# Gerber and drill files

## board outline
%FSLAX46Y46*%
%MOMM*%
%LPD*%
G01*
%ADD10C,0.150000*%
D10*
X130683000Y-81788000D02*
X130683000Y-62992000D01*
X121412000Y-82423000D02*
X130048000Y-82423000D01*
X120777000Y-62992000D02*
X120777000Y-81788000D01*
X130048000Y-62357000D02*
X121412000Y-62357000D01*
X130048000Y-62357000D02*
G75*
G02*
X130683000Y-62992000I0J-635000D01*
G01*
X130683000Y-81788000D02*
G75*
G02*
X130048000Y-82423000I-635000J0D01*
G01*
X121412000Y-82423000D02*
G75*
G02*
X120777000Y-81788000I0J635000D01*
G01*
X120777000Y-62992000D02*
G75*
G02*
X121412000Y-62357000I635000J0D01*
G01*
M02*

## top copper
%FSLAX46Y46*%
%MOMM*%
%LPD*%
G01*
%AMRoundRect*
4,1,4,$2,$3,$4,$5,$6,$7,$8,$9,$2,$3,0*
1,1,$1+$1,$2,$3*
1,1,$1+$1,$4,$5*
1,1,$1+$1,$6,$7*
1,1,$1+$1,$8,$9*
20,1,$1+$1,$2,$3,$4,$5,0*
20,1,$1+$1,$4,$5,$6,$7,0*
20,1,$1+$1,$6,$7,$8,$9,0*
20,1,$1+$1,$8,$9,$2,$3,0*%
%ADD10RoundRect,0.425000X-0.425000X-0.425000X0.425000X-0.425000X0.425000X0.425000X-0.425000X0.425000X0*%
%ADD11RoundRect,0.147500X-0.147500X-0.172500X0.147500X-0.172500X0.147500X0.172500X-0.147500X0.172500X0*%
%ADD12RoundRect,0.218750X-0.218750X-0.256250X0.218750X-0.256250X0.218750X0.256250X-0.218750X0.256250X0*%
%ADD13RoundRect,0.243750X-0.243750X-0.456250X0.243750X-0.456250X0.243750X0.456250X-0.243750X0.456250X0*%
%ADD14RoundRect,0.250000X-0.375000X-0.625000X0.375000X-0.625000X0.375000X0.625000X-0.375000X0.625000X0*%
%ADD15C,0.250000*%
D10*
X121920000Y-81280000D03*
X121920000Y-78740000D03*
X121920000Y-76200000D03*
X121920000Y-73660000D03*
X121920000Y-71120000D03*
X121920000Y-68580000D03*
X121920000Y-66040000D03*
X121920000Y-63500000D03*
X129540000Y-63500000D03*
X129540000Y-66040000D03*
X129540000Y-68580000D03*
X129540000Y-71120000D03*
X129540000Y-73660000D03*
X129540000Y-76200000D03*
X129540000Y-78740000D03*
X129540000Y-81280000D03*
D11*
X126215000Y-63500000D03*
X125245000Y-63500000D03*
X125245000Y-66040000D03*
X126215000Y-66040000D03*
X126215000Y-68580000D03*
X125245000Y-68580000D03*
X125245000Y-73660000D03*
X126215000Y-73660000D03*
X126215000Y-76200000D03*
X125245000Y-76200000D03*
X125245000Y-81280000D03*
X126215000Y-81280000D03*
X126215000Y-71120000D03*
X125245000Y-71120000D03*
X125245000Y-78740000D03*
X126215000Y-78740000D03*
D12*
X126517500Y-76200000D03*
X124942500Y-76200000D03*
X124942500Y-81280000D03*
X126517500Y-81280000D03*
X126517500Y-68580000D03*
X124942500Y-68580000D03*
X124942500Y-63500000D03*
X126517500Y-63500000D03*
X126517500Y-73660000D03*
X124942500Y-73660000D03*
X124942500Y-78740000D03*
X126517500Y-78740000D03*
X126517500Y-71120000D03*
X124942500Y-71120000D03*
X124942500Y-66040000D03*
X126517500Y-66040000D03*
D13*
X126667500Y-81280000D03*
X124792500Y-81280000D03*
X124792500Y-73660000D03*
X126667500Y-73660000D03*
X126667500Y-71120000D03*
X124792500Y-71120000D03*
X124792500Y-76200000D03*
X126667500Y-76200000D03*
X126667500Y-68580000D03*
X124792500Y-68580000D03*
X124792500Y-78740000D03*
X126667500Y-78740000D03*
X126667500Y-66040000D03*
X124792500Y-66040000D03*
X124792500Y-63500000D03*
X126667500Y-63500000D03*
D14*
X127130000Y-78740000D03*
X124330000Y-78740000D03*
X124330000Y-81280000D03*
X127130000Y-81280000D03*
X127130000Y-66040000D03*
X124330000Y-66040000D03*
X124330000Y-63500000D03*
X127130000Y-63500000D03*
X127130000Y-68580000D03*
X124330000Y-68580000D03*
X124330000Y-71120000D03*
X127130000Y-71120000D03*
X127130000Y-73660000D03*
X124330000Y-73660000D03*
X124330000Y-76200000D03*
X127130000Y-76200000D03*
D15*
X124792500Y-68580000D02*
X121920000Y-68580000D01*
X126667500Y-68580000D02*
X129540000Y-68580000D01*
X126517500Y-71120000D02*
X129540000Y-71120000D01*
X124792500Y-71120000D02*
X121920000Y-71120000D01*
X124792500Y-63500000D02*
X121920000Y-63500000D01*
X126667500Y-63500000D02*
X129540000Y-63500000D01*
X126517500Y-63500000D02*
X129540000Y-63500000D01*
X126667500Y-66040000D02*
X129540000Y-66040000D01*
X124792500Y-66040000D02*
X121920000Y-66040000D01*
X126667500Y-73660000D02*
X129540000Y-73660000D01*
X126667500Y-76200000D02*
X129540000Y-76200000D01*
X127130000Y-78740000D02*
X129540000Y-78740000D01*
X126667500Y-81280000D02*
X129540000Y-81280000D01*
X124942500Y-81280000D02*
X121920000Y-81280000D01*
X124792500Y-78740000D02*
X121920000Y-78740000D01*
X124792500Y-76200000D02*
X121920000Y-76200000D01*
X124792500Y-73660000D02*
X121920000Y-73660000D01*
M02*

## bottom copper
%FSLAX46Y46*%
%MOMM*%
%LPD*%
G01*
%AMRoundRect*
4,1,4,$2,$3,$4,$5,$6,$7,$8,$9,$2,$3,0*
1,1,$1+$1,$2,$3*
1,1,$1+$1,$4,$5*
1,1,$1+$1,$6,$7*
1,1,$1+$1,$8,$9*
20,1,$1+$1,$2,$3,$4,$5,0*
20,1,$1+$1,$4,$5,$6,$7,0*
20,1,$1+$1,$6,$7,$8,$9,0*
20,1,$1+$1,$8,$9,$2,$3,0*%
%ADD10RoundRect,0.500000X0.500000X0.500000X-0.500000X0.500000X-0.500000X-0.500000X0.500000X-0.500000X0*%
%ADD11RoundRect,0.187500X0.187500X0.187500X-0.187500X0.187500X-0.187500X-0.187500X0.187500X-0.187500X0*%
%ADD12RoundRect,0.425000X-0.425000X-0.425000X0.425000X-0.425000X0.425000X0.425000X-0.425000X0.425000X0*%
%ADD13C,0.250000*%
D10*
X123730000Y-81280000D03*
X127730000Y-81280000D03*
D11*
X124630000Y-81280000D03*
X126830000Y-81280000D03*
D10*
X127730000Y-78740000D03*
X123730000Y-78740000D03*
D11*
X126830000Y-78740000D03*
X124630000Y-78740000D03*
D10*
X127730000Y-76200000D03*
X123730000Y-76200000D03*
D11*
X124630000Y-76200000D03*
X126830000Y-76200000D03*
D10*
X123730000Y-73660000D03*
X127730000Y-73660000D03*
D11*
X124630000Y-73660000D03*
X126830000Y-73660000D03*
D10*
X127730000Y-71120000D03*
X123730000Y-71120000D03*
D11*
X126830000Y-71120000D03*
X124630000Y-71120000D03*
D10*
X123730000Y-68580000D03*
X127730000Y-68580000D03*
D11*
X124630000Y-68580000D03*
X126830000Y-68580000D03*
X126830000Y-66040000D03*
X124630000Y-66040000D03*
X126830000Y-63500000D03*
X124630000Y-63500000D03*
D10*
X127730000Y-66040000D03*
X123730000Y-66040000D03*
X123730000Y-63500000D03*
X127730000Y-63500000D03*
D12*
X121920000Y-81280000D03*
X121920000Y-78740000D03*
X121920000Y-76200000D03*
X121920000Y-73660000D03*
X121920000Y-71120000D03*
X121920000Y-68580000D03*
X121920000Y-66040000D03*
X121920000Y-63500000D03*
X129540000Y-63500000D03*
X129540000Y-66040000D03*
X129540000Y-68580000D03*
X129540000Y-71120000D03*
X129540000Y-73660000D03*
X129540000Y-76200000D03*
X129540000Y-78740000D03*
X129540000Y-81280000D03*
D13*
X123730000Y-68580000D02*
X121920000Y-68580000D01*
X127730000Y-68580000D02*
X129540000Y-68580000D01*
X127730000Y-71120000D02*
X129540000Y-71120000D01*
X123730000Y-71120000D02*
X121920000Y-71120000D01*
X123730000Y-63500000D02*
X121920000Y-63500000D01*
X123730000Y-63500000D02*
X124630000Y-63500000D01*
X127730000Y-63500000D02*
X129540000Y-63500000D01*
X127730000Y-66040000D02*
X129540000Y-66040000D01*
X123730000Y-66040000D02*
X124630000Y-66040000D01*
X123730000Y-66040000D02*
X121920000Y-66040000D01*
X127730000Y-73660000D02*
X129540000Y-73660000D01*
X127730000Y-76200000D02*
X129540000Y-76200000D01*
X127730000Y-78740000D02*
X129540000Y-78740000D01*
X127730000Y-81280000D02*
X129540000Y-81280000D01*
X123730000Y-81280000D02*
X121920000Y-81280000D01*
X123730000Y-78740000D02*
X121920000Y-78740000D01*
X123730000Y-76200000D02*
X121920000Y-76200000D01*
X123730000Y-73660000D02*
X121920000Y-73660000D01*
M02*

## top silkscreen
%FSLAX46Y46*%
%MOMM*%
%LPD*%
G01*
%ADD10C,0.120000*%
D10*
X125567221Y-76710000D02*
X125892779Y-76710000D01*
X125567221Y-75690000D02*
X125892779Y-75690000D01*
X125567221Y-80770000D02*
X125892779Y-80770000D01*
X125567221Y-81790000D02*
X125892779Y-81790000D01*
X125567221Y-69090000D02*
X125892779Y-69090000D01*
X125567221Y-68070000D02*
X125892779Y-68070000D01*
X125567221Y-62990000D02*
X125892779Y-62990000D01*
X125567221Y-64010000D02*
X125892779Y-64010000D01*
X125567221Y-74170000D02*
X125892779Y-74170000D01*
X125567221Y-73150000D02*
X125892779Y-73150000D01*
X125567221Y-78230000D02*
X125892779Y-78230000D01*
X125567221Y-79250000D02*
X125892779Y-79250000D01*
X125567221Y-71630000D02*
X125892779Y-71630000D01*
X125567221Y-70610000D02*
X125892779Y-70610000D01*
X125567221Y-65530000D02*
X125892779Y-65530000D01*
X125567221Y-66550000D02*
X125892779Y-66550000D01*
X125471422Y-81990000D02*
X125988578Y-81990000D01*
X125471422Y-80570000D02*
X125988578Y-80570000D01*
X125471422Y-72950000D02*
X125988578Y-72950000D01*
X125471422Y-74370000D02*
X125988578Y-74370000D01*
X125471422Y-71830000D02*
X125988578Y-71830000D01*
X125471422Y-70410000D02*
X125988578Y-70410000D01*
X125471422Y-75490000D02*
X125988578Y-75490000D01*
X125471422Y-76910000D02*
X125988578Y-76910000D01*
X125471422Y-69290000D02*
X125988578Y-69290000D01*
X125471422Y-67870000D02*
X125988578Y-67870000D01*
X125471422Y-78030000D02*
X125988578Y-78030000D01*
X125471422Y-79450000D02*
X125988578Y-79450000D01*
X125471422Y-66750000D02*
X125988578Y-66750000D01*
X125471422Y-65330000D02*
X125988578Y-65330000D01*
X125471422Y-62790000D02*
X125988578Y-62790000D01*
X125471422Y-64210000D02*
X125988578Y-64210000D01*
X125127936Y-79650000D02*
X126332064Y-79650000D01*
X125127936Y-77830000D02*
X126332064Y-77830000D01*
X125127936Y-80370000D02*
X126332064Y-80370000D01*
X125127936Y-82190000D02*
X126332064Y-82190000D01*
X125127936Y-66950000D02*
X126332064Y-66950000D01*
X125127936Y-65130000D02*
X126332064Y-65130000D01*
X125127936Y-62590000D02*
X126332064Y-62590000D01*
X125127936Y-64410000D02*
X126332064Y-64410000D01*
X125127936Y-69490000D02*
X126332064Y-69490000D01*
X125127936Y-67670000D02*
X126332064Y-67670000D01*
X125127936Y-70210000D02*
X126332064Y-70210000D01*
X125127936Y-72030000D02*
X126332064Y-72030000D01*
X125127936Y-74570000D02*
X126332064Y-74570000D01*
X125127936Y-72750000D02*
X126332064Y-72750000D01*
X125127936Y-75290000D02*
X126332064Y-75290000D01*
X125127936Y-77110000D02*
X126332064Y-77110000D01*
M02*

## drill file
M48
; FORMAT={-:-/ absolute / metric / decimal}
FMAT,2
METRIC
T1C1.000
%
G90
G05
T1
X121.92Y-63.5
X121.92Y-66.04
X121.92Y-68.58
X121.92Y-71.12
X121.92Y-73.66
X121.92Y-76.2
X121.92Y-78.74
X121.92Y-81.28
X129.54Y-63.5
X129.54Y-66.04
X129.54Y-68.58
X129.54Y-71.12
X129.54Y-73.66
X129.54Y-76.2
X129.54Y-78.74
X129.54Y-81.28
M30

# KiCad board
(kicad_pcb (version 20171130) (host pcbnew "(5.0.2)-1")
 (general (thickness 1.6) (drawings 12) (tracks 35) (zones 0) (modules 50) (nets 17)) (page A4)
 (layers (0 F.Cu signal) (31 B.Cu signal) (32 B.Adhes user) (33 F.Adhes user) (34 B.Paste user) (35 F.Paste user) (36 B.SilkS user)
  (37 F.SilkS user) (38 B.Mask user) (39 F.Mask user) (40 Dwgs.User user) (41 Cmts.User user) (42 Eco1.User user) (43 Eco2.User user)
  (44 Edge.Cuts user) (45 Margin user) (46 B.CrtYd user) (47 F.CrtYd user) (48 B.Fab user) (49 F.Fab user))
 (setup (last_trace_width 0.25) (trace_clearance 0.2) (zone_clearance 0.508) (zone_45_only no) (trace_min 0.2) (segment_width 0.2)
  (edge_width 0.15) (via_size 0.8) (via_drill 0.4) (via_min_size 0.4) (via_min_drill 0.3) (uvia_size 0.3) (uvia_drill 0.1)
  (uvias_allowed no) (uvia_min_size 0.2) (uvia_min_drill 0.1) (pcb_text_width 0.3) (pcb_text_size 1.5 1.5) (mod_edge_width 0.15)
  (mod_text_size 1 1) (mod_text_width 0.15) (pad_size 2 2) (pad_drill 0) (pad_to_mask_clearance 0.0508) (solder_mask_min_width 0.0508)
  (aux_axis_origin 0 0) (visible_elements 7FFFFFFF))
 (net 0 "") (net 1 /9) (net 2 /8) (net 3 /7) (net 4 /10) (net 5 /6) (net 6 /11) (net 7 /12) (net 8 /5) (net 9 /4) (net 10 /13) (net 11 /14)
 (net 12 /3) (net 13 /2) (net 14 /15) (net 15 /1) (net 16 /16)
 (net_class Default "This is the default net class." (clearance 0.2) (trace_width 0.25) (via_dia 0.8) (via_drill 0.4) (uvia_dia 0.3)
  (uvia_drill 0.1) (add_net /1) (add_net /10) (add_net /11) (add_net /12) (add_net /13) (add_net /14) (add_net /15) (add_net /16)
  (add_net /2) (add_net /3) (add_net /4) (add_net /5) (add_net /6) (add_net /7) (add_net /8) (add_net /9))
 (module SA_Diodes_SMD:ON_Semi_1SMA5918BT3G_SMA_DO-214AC (layer B.Cu) (at 125.73 81.28 180)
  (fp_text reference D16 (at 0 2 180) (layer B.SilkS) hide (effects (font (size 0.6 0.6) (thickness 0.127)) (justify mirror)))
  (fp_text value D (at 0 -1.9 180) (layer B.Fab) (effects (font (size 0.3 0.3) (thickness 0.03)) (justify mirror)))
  (pad 2 smd roundrect (at 2 0 180) (size 2 2) (layers B.Cu B.Paste B.Mask) (roundrect_rratio 0.25) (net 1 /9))
  (pad 1 smd roundrect (at -2 0 180) (size 2 2) (layers B.Cu B.Paste B.Mask) (roundrect_rratio 0.25) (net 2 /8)))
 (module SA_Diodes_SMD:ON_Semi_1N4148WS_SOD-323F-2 (layer B.Cu) (at 125.73 81.28 180)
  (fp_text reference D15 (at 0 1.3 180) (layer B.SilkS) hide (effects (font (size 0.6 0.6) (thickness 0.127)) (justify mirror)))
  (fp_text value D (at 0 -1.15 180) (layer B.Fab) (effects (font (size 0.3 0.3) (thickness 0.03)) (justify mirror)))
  (pad 2 smd roundrect (at 1.1 0 180) (size 0.75 0.75) (layers B.Cu B.Paste B.Mask) (roundrect_rratio 0.25) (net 1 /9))
  (pad 1 smd roundrect (at -1.1 0 180) (size 0.75 0.75) (layers B.Cu B.Paste B.Mask) (roundrect_rratio 0.25) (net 2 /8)))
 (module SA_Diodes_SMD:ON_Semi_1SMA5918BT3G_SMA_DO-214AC (layer B.Cu) (at 125.73 78.74 180)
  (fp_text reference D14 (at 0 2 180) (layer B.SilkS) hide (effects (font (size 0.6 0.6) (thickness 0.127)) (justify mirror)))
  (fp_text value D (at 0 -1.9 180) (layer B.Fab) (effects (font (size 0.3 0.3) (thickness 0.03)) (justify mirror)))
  (pad 1 smd roundrect (at -2 0 180) (size 2 2) (layers B.Cu B.Paste B.Mask) (roundrect_rratio 0.25) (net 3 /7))
  (pad 2 smd roundrect (at 2 0 180) (size 2 2) (layers B.Cu B.Paste B.Mask) (roundrect_rratio 0.25) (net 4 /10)))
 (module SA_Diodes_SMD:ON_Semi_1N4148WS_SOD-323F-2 (layer B.Cu) (at 125.73 78.74 180)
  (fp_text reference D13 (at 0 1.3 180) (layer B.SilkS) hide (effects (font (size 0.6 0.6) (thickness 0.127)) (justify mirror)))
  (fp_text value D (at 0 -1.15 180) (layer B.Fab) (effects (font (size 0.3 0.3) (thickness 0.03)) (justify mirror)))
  (pad 1 smd roundrect (at -1.1 0 180) (size 0.75 0.75) (layers B.Cu B.Paste B.Mask) (roundrect_rratio 0.25) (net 3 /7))
  (pad 2 smd roundrect (at 1.1 0 180) (size 0.75 0.75) (layers B.Cu B.Paste B.Mask) (roundrect_rratio 0.25) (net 4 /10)))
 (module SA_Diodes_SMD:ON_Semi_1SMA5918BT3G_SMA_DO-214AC (layer B.Cu) (at 125.73 76.2 180)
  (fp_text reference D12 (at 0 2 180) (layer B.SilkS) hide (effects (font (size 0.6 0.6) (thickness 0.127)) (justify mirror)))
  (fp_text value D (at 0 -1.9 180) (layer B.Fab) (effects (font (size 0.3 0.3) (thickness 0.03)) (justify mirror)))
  (pad 1 smd roundrect (at -2 0 180) (size 2 2) (layers B.Cu B.Paste B.Mask) (roundrect_rratio 0.25) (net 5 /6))
  (pad 2 smd roundrect (at 2 0 180) (size 2 2) (layers B.Cu B.Paste B.Mask) (roundrect_rratio 0.25) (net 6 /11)))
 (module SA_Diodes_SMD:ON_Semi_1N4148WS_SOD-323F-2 (layer B.Cu) (at 125.73 76.2 180)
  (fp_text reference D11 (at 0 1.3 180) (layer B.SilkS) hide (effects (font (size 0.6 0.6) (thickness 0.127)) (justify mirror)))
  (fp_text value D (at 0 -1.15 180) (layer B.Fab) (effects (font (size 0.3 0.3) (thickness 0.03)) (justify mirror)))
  (pad 2 smd roundrect (at 1.1 0 180) (size 0.75 0.75) (layers B.Cu B.Paste B.Mask) (roundrect_rratio 0.25) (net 6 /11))
  (pad 1 smd roundrect (at -1.1 0 180) (size 0.75 0.75) (layers B.Cu B.Paste B.Mask) (roundrect_rratio 0.25) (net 5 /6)))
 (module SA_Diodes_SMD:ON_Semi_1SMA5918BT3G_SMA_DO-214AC (layer B.Cu) (at 125.73 73.66 180)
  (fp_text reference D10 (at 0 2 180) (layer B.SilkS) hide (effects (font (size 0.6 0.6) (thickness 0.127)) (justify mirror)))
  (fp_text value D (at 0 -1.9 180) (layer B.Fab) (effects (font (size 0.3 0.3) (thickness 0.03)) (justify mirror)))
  (pad 2 smd roundrect (at 2 0 180) (size 2 2) (layers B.Cu B.Paste B.Mask) (roundrect_rratio 0.25) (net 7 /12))
  (pad 1 smd roundrect (at -2 0 180) (size 2 2) (layers B.Cu B.Paste B.Mask) (roundrect_rratio 0.25) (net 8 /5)))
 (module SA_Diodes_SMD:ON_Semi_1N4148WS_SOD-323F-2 (layer B.Cu) (at 125.73 73.66 180)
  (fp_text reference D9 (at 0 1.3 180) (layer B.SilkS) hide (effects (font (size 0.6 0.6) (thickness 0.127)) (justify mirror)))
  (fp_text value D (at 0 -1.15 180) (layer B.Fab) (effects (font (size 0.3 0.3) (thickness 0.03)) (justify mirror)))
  (pad 2 smd roundrect (at 1.1 0 180) (size 0.75 0.75) (layers B.Cu B.Paste B.Mask) (roundrect_rratio 0.25) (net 7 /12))
  (pad 1 smd roundrect (at -1.1 0 180) (size 0.75 0.75) (layers B.Cu B.Paste B.Mask) (roundrect_rratio 0.25) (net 8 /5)))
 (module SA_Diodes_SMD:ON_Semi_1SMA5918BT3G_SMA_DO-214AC (layer B.Cu) (at 125.73 71.12 180)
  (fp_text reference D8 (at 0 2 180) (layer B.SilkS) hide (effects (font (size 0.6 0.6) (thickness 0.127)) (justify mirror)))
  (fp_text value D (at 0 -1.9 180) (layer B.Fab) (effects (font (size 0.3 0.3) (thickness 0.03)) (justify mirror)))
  (pad 1 smd roundrect (at -2 0 180) (size 2 2) (layers B.Cu B.Paste B.Mask) (roundrect_rratio 0.25) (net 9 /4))
  (pad 2 smd roundrect (at 2 0 180) (size 2 2) (layers B.Cu B.Paste B.Mask) (roundrect_rratio 0.25) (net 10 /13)))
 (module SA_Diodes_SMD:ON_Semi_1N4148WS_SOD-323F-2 (layer B.Cu) (at 125.73 71.12 180)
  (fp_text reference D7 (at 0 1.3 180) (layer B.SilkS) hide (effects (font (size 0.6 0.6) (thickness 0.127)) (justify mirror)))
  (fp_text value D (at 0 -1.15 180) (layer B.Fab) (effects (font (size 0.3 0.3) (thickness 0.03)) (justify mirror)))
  (pad 1 smd roundrect (at -1.1 0 180) (size 0.75 0.75) (layers B.Cu B.Paste B.Mask) (roundrect_rratio 0.25) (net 9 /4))
  (pad 2 smd roundrect (at 1.1 0 180) (size 0.75 0.75) (layers B.Cu B.Paste B.Mask) (roundrect_rratio 0.25) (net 10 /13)))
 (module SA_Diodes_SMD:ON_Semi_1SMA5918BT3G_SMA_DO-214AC (layer B.Cu) (at 125.73 68.58 180)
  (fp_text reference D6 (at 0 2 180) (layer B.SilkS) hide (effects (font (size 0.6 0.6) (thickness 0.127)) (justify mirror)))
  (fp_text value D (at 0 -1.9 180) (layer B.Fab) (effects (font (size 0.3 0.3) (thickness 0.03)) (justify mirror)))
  (pad 2 smd roundrect (at 2 0 180) (size 2 2) (layers B.Cu B.Paste B.Mask) (roundrect_rratio 0.25) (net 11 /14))
  (pad 1 smd roundrect (at -2 0 180) (size 2 2) (layers B.Cu B.Paste B.Mask) (roundrect_rratio 0.25) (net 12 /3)))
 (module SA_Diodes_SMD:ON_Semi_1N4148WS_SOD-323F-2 (layer B.Cu) (at 125.73 68.58 180)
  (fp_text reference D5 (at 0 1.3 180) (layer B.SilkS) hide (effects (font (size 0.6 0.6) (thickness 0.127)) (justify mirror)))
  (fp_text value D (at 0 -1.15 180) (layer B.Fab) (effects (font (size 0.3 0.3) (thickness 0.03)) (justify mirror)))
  (pad 2 smd roundrect (at 1.1 0 180) (size 0.75 0.75) (layers B.Cu B.Paste B.Mask) (roundrect_rratio 0.25) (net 11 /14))
  (pad 1 smd roundrect (at -1.1 0 180) (size 0.75 0.75) (layers B.Cu B.Paste B.Mask) (roundrect_rratio 0.25) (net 12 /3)))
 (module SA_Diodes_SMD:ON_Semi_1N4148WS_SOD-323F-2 (layer B.Cu) (at 125.73 66.04 180)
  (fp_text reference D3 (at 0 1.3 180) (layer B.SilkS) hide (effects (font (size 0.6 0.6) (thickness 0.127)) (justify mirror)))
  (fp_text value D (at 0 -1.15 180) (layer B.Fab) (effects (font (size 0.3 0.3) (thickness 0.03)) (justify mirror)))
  (pad 1 smd roundrect (at -1.1 0 180) (size 0.75 0.75) (layers B.Cu B.Paste B.Mask) (roundrect_rratio 0.25) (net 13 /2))
  (pad 2 smd roundrect (at 1.1 0 180) (size 0.75 0.75) (layers B.Cu B.Paste B.Mask) (roundrect_rratio 0.25) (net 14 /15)))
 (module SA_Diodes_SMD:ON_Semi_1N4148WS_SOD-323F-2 (layer B.Cu) (at 125.73 63.5 180)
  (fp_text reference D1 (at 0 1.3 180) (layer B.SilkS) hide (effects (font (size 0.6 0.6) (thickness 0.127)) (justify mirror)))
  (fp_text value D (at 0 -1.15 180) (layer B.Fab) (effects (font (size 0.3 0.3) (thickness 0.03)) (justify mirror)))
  (pad 1 smd roundrect (at -1.1 0 180) (size 0.75 0.75) (layers B.Cu B.Paste B.Mask) (roundrect_rratio 0.25) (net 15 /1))
  (pad 2 smd roundrect (at 1.1 0 180) (size 0.75 0.75) (layers B.Cu B.Paste B.Mask) (roundrect_rratio 0.25) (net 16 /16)))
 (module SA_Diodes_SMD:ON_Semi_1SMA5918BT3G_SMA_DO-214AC (layer B.Cu) (at 125.73 66.04 180)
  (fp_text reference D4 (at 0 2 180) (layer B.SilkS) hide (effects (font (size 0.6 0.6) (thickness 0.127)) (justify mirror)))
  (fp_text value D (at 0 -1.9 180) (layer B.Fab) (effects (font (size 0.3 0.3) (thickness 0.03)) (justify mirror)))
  (pad 1 smd roundrect (at -2 0 180) (size 2 2) (layers B.Cu B.Paste B.Mask) (roundrect_rratio 0.25) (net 13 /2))
  (pad 2 smd roundrect (at 2 0 180) (size 2 2) (layers B.Cu B.Paste B.Mask) (roundrect_rratio 0.25) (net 14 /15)))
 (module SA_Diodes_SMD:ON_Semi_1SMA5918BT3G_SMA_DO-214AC (layer B.Cu) (at 125.73 63.5 180)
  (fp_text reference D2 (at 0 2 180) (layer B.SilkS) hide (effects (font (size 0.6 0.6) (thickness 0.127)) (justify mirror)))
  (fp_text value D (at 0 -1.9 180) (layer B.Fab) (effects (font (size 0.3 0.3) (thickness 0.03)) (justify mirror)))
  (pad 2 smd roundrect (at 2 0 180) (size 2 2) (layers B.Cu B.Paste B.Mask) (roundrect_rratio 0.25) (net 16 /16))
  (pad 1 smd roundrect (at -2 0 180) (size 2 2) (layers B.Cu B.Paste B.Mask) (roundrect_rratio 0.25) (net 15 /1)))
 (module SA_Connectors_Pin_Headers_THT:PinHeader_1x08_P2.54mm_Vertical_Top (layer F.Cu) (at 121.92 63.5)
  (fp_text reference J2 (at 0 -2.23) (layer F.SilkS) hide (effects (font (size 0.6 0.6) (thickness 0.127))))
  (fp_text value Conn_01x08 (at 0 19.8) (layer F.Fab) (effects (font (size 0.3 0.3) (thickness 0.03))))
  (pad 8 thru_hole roundrect (at 0 17.78) (size 1.7 1.7) (drill 1) (layers *.Cu *.Mask) (roundrect_rratio 0.25) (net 1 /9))
  (pad 7 thru_hole roundrect (at 0 15.24) (size 1.7 1.7) (drill 1) (layers *.Cu *.Mask) (roundrect_rratio 0.25) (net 4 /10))
  (pad 6 thru_hole roundrect (at 0 12.7) (size 1.7 1.7) (drill 1) (layers *.Cu *.Mask) (roundrect_rratio 0.25) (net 6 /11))
  (pad 5 thru_hole roundrect (at 0 10.16) (size 1.7 1.7) (drill 1) (layers *.Cu *.Mask) (roundrect_rratio 0.25) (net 7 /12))
  (pad 4 thru_hole roundrect (at 0 7.62) (size 1.7 1.7) (drill 1) (layers *.Cu *.Mask) (roundrect_rratio 0.25) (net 10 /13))
  (pad 3 thru_hole roundrect (at 0 5.08) (size 1.7 1.7) (drill 1) (layers *.Cu *.Mask) (roundrect_rratio 0.25) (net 11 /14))
  (pad 2 thru_hole roundrect (at 0 2.54) (size 1.7 1.7) (drill 1) (layers *.Cu *.Mask) (roundrect_rratio 0.25) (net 14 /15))
  (pad 1 thru_hole roundrect (at 0 0) (size 1.7 1.7) (drill 1) (layers *.Cu *.Mask) (roundrect_rratio 0.25) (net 16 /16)))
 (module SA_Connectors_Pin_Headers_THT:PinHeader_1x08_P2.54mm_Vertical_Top (layer F.Cu) (at 129.54 63.5)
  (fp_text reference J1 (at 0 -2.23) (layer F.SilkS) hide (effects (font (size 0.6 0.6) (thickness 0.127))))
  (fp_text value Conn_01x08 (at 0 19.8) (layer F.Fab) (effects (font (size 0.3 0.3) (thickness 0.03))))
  (pad 1 thru_hole roundrect (at 0 0) (size 1.7 1.7) (drill 1) (layers *.Cu *.Mask) (roundrect_rratio 0.25) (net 15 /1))
  (pad 2 thru_hole roundrect (at 0 2.54) (size 1.7 1.7) (drill 1) (layers *.Cu *.Mask) (roundrect_rratio 0.25) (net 13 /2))
  (pad 3 thru_hole roundrect (at 0 5.08) (size 1.7 1.7) (drill 1) (layers *.Cu *.Mask) (roundrect_rratio 0.25) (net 12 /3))
  (pad 4 thru_hole roundrect (at 0 7.62) (size 1.7 1.7) (drill 1) (layers *.Cu *.Mask) (roundrect_rratio 0.25) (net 9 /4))
  (pad 5 thru_hole roundrect (at 0 10.16) (size 1.7 1.7) (drill 1) (layers *.Cu *.Mask) (roundrect_rratio 0.25) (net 8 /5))
  (pad 6 thru_hole roundrect (at 0 12.7) (size 1.7 1.7) (drill 1) (layers *.Cu *.Mask) (roundrect_rratio 0.25) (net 5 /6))
  (pad 7 thru_hole roundrect (at 0 15.24) (size 1.7 1.7) (drill 1) (layers *.Cu *.Mask) (roundrect_rratio 0.25) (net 3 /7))
  (pad 8 thru_hole roundrect (at 0 17.78) (size 1.7 1.7) (drill 1) (layers *.Cu *.Mask) (roundrect_rratio 0.25) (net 2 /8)))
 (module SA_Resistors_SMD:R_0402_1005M (layer F.Cu) (at 125.73 63.5)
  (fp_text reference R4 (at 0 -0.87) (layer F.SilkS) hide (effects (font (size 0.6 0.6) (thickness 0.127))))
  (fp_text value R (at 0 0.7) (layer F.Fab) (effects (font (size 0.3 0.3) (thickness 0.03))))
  (pad 2 smd roundrect (at 0.485 0) (size 0.59 0.64) (layers F.Cu F.Paste F.Mask) (roundrect_rratio 0.25) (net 15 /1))
  (pad 1 smd roundrect (at -0.485 0) (size 0.59 0.64) (layers F.Cu F.Paste F.Mask) (roundrect_rratio 0.25) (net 16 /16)))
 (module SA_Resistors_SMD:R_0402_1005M (layer F.Cu) (at 125.73 66.04)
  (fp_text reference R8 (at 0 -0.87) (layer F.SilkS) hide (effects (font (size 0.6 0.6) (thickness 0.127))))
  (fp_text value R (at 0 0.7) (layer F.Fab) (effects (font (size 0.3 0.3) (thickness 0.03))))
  (pad 1 smd roundrect (at -0.485 0) (size 0.59 0.64) (layers F.Cu F.Paste F.Mask) (roundrect_rratio 0.25) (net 14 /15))
  (pad 2 smd roundrect (at 0.485 0) (size 0.59 0.64) (layers F.Cu F.Paste F.Mask) (roundrect_rratio 0.25) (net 13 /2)))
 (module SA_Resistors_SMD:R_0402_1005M (layer F.Cu) (at 125.73 68.58)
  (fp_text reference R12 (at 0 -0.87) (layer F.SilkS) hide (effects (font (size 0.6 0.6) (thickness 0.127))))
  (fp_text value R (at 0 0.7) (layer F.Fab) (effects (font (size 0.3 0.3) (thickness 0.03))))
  (pad 2 smd roundrect (at 0.485 0) (size 0.59 0.64) (layers F.Cu F.Paste F.Mask) (roundrect_rratio 0.25) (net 12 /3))
  (pad 1 smd roundrect (at -0.485 0) (size 0.59 0.64) (layers F.Cu F.Paste F.Mask) (roundrect_rratio 0.25) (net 11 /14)))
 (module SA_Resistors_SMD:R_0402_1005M (layer F.Cu) (at 125.73 73.66)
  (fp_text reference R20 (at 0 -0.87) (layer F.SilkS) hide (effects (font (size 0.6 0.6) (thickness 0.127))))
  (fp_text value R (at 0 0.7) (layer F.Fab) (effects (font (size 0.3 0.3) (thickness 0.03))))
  (pad 1 smd roundrect (at -0.485 0) (size 0.59 0.64) (layers F.Cu F.Paste F.Mask) (roundrect_rratio 0.25) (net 7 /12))
  (pad 2 smd roundrect (at 0.485 0) (size 0.59 0.64) (layers F.Cu F.Paste F.Mask) (roundrect_rratio 0.25) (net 8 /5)))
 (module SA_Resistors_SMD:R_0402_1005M (layer F.Cu) (at 125.73 76.2)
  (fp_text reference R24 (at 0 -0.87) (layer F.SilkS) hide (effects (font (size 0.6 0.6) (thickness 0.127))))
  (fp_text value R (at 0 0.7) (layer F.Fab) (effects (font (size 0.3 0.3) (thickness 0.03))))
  (pad 2 smd roundrect (at 0.485 0) (size 0.59 0.64) (layers F.Cu F.Paste F.Mask) (roundrect_rratio 0.25) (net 5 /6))
  (pad 1 smd roundrect (at -0.485 0) (size 0.59 0.64) (layers F.Cu F.Paste F.Mask) (roundrect_rratio 0.25) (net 6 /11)))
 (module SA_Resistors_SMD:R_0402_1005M (layer F.Cu) (at 125.73 81.28)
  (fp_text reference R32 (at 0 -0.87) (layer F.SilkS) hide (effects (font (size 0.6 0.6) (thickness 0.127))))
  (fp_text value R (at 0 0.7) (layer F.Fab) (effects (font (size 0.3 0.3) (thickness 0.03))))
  (pad 1 smd roundrect (at -0.485 0) (size 0.59 0.64) (layers F.Cu F.Paste F.Mask) (roundrect_rratio 0.25) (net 1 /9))
  (pad 2 smd roundrect (at 0.485 0) (size 0.59 0.64) (layers F.Cu F.Paste F.Mask) (roundrect_rratio 0.25) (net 2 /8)))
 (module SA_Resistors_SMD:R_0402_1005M (layer F.Cu) (at 125.73 71.12)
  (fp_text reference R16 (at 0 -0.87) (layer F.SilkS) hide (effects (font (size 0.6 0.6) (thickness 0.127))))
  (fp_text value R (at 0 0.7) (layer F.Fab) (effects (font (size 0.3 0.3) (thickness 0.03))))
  (pad 2 smd roundrect (at 0.485 0) (size 0.59 0.64) (layers F.Cu F.Paste F.Mask) (roundrect_rratio 0.25) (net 9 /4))
  (pad 1 smd roundrect (at -0.485 0) (size 0.59 0.64) (layers F.Cu F.Paste F.Mask) (roundrect_rratio 0.25) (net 10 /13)))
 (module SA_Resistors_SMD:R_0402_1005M (layer F.Cu) (at 125.73 78.74)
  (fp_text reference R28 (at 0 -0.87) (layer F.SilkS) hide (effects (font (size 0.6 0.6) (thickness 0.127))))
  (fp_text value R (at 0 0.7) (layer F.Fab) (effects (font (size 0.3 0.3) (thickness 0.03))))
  (pad 1 smd roundrect (at -0.485 0) (size 0.59 0.64) (layers F.Cu F.Paste F.Mask) (roundrect_rratio 0.25) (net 4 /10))
  (pad 2 smd roundrect (at 0.485 0) (size 0.59 0.64) (layers F.Cu F.Paste F.Mask) (roundrect_rratio 0.25) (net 3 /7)))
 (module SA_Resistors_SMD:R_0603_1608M (layer F.Cu) (at 125.73 76.2)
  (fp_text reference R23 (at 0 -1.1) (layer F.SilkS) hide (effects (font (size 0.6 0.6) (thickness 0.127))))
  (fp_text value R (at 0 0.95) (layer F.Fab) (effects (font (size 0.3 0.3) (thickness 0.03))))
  (fp_line (start -0.162779 0.51) (end 0.162779 0.51) (layer F.SilkS) (width 0.12))
  (fp_line (start -0.162779 -0.51) (end 0.162779 -0.51) (layer F.SilkS) (width 0.12))
  (pad 2 smd roundrect (at 0.7875 0) (size 0.875 0.95) (layers F.Cu F.Paste F.Mask) (roundrect_rratio 0.25) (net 5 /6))
  (pad 1 smd roundrect (at -0.7875 0) (size 0.875 0.95) (layers F.Cu F.Paste F.Mask) (roundrect_rratio 0.25) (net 6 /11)))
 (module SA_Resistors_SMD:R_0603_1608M (layer F.Cu) (at 125.73 81.28)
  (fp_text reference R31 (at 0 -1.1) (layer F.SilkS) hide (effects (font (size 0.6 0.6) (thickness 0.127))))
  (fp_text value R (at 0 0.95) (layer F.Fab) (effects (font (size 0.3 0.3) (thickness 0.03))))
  (fp_line (start -0.162779 -0.51) (end 0.162779 -0.51) (layer F.SilkS) (width 0.12))
  (fp_line (start -0.162779 0.51) (end 0.162779 0.51) (layer F.SilkS) (width 0.12))
  (pad 1 smd roundrect (at -0.7875 0) (size 0.875 0.95) (layers F.Cu F.Paste F.Mask) (roundrect_rratio 0.25) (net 1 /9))
  (pad 2 smd roundrect (at 0.7875 0) (size 0.875 0.95) (layers F.Cu F.Paste F.Mask) (roundrect_rratio 0.25) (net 2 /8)))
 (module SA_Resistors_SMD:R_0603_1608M (layer F.Cu) (at 125.73 68.58)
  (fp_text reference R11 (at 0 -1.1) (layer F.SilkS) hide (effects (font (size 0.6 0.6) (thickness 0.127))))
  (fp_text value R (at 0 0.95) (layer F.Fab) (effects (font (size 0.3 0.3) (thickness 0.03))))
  (fp_line (start -0.162779 0.51) (end 0.162779 0.51) (layer F.SilkS) (width 0.12))
  (fp_line (start -0.162779 -0.51) (end 0.162779 -0.51) (layer F.SilkS) (width 0.12))
  (pad 2 smd roundrect (at 0.7875 0) (size 0.875 0.95) (layers F.Cu F.Paste F.Mask) (roundrect_rratio 0.25) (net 12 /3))
  (pad 1 smd roundrect (at -0.7875 0) (size 0.875 0.95) (layers F.Cu F.Paste F.Mask) (roundrect_rratio 0.25) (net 11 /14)))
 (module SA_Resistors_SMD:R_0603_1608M (layer F.Cu) (at 125.73 63.5)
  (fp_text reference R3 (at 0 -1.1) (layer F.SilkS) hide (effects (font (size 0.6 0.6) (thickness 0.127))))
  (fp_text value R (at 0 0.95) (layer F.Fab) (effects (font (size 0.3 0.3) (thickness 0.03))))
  (fp_line (start -0.162779 -0.51) (end 0.162779 -0.51) (layer F.SilkS) (width 0.12))
  (fp_line (start -0.162779 0.51) (end 0.162779 0.51) (layer F.SilkS) (width 0.12))
  (pad 1 smd roundrect (at -0.7875 0) (size 0.875 0.95) (layers F.Cu F.Paste F.Mask) (roundrect_rratio 0.25) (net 16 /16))
  (pad 2 smd roundrect (at 0.7875 0) (size 0.875 0.95) (layers F.Cu F.Paste F.Mask) (roundrect_rratio 0.25) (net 15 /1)))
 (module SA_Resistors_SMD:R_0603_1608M (layer F.Cu) (at 125.73 73.66)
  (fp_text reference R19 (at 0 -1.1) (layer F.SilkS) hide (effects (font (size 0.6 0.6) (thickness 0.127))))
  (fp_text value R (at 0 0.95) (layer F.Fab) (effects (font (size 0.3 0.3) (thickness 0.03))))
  (fp_line (start -0.162779 0.51) (end 0.162779 0.51) (layer F.SilkS) (width 0.12))
  (fp_line (start -0.162779 -0.51) (end 0.162779 -0.51) (layer F.SilkS) (width 0.12))
  (pad 2 smd roundrect (at 0.7875 0) (size 0.875 0.95) (layers F.Cu F.Paste F.Mask) (roundrect_rratio 0.25) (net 8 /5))
  (pad 1 smd roundrect (at -0.7875 0) (size 0.875 0.95) (layers F.Cu F.Paste F.Mask) (roundrect_rratio 0.25) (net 7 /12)))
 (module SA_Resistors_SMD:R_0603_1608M (layer F.Cu) (at 125.73 78.74)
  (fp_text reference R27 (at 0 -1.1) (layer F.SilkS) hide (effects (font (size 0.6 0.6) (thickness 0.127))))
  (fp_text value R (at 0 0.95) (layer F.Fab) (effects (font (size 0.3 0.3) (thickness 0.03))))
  (fp_line (start -0.162779 -0.51) (end 0.162779 -0.51) (layer F.SilkS) (width 0.12))
  (fp_line (start -0.162779 0.51) (end 0.162779 0.51) (layer F.SilkS) (width 0.12))
  (pad 1 smd roundrect (at -0.7875 0) (size 0.875 0.95) (layers F.Cu F.Paste F.Mask) (roundrect_rratio 0.25) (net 4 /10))
  (pad 2 smd roundrect (at 0.7875 0) (size 0.875 0.95) (layers F.Cu F.Paste F.Mask) (roundrect_rratio 0.25) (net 3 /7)))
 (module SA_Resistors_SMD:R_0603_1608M (layer F.Cu) (at 125.73 71.12)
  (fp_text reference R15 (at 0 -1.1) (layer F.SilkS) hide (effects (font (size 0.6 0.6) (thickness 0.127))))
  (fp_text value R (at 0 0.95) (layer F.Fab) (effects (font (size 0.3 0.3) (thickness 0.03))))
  (fp_line (start -0.162779 0.51) (end 0.162779 0.51) (layer F.SilkS) (width 0.12))
  (fp_line (start -0.162779 -0.51) (end 0.162779 -0.51) (layer F.SilkS) (width 0.12))
  (pad 2 smd roundrect (at 0.7875 0) (size 0.875 0.95) (layers F.Cu F.Paste F.Mask) (roundrect_rratio 0.25) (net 9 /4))
  (pad 1 smd roundrect (at -0.7875 0) (size 0.875 0.95) (layers F.Cu F.Paste F.Mask) (roundrect_rratio 0.25) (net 10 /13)))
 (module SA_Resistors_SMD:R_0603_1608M (layer F.Cu) (at 125.73 66.04)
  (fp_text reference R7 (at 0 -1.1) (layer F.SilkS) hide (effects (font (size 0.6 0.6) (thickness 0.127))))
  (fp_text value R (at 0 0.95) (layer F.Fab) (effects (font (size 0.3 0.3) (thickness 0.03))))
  (fp_line (start -0.162779 -0.51) (end 0.162779 -0.51) (layer F.SilkS) (width 0.12))
  (fp_line (start -0.162779 0.51) (end 0.162779 0.51) (layer F.SilkS) (width 0.12))
  (pad 1 smd roundrect (at -0.7875 0) (size 0.875 0.95) (layers F.Cu F.Paste F.Mask) (roundrect_rratio 0.25) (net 14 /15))
  (pad 2 smd roundrect (at 0.7875 0) (size 0.875 0.95) (layers F.Cu F.Paste F.Mask) (roundrect_rratio 0.25) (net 13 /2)))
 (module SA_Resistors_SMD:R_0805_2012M (layer F.Cu) (at 125.73 81.28)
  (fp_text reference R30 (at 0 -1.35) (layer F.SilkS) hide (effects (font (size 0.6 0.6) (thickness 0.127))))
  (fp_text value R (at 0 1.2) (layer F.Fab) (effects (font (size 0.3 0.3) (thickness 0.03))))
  (fp_line (start -0.258578 0.71) (end 0.258578 0.71) (layer F.SilkS) (width 0.12))
  (fp_line (start -0.258578 -0.71) (end 0.258578 -0.71) (layer F.SilkS) (width 0.12))
  (pad 2 smd roundrect (at 0.9375 0) (size 0.975 1.4) (layers F.Cu F.Paste F.Mask) (roundrect_rratio 0.25) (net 2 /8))
  (pad 1 smd roundrect (at -0.9375 0) (size 0.975 1.4) (layers F.Cu F.Paste F.Mask) (roundrect_rratio 0.25) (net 1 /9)))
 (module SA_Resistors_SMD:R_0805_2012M (layer F.Cu) (at 125.73 73.66)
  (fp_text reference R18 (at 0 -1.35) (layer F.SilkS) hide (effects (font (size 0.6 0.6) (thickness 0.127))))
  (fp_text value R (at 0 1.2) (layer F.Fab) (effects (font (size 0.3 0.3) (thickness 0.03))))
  (fp_line (start -0.258578 -0.71) (end 0.258578 -0.71) (layer F.SilkS) (width 0.12))
  (fp_line (start -0.258578 0.71) (end 0.258578 0.71) (layer F.SilkS) (width 0.12))
  (pad 1 smd roundrect (at -0.9375 0) (size 0.975 1.4) (layers F.Cu F.Paste F.Mask) (roundrect_rratio 0.25) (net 7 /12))
  (pad 2 smd roundrect (at 0.9375 0) (size 0.975 1.4) (layers F.Cu F.Paste F.Mask) (roundrect_rratio 0.25) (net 8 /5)))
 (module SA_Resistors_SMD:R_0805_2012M (layer F.Cu) (at 125.73 71.12)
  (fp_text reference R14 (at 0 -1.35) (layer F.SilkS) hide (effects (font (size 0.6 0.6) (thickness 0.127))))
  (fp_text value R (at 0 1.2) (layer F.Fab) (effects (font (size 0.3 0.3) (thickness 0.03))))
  (fp_line (start -0.258578 0.71) (end 0.258578 0.71) (layer F.SilkS) (width 0.12))
  (fp_line (start -0.258578 -0.71) (end 0.258578 -0.71) (layer F.SilkS) (width 0.12))
  (pad 2 smd roundrect (at 0.9375 0) (size 0.975 1.4) (layers F.Cu F.Paste F.Mask) (roundrect_rratio 0.25) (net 9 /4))
  (pad 1 smd roundrect (at -0.9375 0) (size 0.975 1.4) (layers F.Cu F.Paste F.Mask) (roundrect_rratio 0.25) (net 10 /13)))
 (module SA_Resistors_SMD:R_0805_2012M (layer F.Cu) (at 125.73 76.2)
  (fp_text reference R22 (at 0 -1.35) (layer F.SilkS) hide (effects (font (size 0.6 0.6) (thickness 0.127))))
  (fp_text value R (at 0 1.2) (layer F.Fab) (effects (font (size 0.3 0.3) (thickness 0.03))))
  (fp_line (start -0.258578 -0.71) (end 0.258578 -0.71) (layer F.SilkS) (width 0.12))
  (fp_line (start -0.258578 0.71) (end 0.258578 0.71) (layer F.SilkS) (width 0.12))
  (pad 1 smd roundrect (at -0.9375 0) (size 0.975 1.4) (layers F.Cu F.Paste F.Mask) (roundrect_rratio 0.25) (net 6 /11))
  (pad 2 smd roundrect (at 0.9375 0) (size 0.975 1.4) (layers F.Cu F.Paste F.Mask) (roundrect_rratio 0.25) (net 5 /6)))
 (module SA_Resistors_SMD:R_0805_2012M (layer F.Cu) (at 125.73 68.58)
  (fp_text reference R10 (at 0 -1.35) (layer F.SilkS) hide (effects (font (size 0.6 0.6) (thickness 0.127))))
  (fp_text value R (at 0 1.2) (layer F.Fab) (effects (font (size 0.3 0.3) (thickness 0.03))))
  (fp_line (start -0.258578 0.71) (end 0.258578 0.71) (layer F.SilkS) (width 0.12))
  (fp_line (start -0.258578 -0.71) (end 0.258578 -0.71) (layer F.SilkS) (width 0.12))
  (pad 2 smd roundrect (at 0.9375 0) (size 0.975 1.4) (layers F.Cu F.Paste F.Mask) (roundrect_rratio 0.25) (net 12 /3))
  (pad 1 smd roundrect (at -0.9375 0) (size 0.975 1.4) (layers F.Cu F.Paste F.Mask) (roundrect_rratio 0.25) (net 11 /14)))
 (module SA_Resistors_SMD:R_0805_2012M (layer F.Cu) (at 125.73 78.74)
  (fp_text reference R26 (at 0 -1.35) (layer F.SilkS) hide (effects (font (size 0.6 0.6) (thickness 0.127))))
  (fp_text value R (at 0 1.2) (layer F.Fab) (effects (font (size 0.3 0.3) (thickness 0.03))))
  (fp_line (start -0.258578 -0.71) (end 0.258578 -0.71) (layer F.SilkS) (width 0.12))
  (fp_line (start -0.258578 0.71) (end 0.258578 0.71) (layer F.SilkS) (width 0.12))
  (pad 1 smd roundrect (at -0.9375 0) (size 0.975 1.4) (layers F.Cu F.Paste F.Mask) (roundrect_rratio 0.25) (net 4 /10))
  (pad 2 smd roundrect (at 0.9375 0) (size 0.975 1.4) (layers F.Cu F.Paste F.Mask) (roundrect_rratio 0.25) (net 3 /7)))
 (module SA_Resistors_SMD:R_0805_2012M (layer F.Cu) (at 125.73 66.04)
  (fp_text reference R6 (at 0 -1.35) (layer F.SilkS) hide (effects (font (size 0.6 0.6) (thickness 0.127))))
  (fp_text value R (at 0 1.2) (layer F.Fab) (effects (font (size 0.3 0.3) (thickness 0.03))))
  (fp_line (start -0.258578 0.71) (end 0.258578 0.71) (layer F.SilkS) (width 0.12))
  (fp_line (start -0.258578 -0.71) (end 0.258578 -0.71) (layer F.SilkS) (width 0.12))
  (pad 2 smd roundrect (at 0.9375 0) (size 0.975 1.4) (layers F.Cu F.Paste F.Mask) (roundrect_rratio 0.25) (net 13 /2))
  (pad 1 smd roundrect (at -0.9375 0) (size 0.975 1.4) (layers F.Cu F.Paste F.Mask) (roundrect_rratio 0.25) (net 14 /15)))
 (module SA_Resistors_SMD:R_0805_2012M (layer F.Cu) (at 125.73 63.5)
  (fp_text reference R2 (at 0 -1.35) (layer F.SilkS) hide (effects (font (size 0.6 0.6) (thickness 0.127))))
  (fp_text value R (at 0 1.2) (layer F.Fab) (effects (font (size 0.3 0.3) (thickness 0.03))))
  (fp_line (start -0.258578 -0.71) (end 0.258578 -0.71) (layer F.SilkS) (width 0.12))
  (fp_line (start -0.258578 0.71) (end 0.258578 0.71) (layer F.SilkS) (width 0.12))
  (pad 1 smd roundrect (at -0.9375 0) (size 0.975 1.4) (layers F.Cu F.Paste F.Mask) (roundrect_rratio 0.25) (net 16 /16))
  (pad 2 smd roundrect (at 0.9375 0) (size 0.975 1.4) (layers F.Cu F.Paste F.Mask) (roundrect_rratio 0.25) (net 15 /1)))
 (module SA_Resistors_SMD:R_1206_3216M (layer F.Cu) (at 125.73 78.74)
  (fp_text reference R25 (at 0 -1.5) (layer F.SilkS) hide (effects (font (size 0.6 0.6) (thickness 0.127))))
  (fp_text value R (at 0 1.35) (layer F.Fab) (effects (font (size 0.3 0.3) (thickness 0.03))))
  (fp_line (start -0.602064 0.91) (end 0.602064 0.91) (layer F.SilkS) (width 0.12))
  (fp_line (start -0.602064 -0.91) (end 0.602064 -0.91) (layer F.SilkS) (width 0.12))
  (pad 2 smd roundrect (at 1.4 0) (size 1.25 1.75) (layers F.Cu F.Paste F.Mask) (roundrect_rratio 0.2) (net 3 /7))
  (pad 1 smd roundrect (at -1.4 0) (size 1.25 1.75) (layers F.Cu F.Paste F.Mask) (roundrect_rratio 0.2) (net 4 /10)))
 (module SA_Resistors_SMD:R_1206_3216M (layer F.Cu) (at 125.73 81.28)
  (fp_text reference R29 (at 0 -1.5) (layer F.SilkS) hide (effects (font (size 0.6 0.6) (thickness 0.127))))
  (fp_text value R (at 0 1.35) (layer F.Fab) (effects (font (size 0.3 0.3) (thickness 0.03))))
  (fp_line (start -0.602064 -0.91) (end 0.602064 -0.91) (layer F.SilkS) (width 0.12))
  (fp_line (start -0.602064 0.91) (end 0.602064 0.91) (layer F.SilkS) (width 0.12))
  (pad 1 smd roundrect (at -1.4 0) (size 1.25 1.75) (layers F.Cu F.Paste F.Mask) (roundrect_rratio 0.2) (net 1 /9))
  (pad 2 smd roundrect (at 1.4 0) (size 1.25 1.75) (layers F.Cu F.Paste F.Mask) (roundrect_rratio 0.2) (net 2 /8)))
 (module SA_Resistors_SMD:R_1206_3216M (layer F.Cu) (at 125.73 66.04)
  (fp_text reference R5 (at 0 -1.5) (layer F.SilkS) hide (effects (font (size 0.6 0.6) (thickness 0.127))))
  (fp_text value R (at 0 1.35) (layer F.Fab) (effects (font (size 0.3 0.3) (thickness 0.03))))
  (fp_line (start -0.602064 0.91) (end 0.602064 0.91) (layer F.SilkS) (width 0.12))
  (fp_line (start -0.602064 -0.91) (end 0.602064 -0.91) (layer F.SilkS) (width 0.12))
  (pad 2 smd roundrect (at 1.4 0) (size 1.25 1.75) (layers F.Cu F.Paste F.Mask) (roundrect_rratio 0.2) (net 13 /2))
  (pad 1 smd roundrect (at -1.4 0) (size 1.25 1.75) (layers F.Cu F.Paste F.Mask) (roundrect_rratio 0.2) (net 14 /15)))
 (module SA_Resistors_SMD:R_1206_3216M (layer F.Cu) (at 125.73 63.5)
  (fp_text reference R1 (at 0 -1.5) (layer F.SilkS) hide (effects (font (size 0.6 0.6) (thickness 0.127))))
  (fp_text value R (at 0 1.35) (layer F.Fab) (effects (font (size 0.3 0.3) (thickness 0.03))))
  (fp_line (start -0.602064 -0.91) (end 0.602064 -0.91) (layer F.SilkS) (width 0.12))
  (fp_line (start -0.602064 0.91) (end 0.602064 0.91) (layer F.SilkS) (width 0.12))
  (pad 1 smd roundrect (at -1.4 0) (size 1.25 1.75) (layers F.Cu F.Paste F.Mask) (roundrect_rratio 0.2) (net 16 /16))
  (pad 2 smd roundrect (at 1.4 0) (size 1.25 1.75) (layers F.Cu F.Paste F.Mask) (roundrect_rratio 0.2) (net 15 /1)))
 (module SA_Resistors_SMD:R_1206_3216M (layer F.Cu) (at 125.73 68.58)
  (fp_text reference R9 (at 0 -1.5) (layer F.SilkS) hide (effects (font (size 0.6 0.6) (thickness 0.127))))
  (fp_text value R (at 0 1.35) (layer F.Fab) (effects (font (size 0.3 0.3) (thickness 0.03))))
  (fp_line (start -0.602064 0.91) (end 0.602064 0.91) (layer F.SilkS) (width 0.12))
  (fp_line (start -0.602064 -0.91) (end 0.602064 -0.91) (layer F.SilkS) (width 0.12))
  (pad 2 smd roundrect (at 1.4 0) (size 1.25 1.75) (layers F.Cu F.Paste F.Mask) (roundrect_rratio 0.2) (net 12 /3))
  (pad 1 smd roundrect (at -1.4 0) (size 1.25 1.75) (layers F.Cu F.Paste F.Mask) (roundrect_rratio 0.2) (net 11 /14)))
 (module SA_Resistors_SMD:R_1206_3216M (layer F.Cu) (at 125.73 71.12)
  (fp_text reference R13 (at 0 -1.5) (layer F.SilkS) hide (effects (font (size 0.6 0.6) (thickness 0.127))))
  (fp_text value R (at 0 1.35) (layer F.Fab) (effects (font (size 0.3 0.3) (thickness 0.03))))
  (fp_line (start -0.602064 -0.91) (end 0.602064 -0.91) (layer F.SilkS) (width 0.12))
  (fp_line (start -0.602064 0.91) (end 0.602064 0.91) (layer F.SilkS) (width 0.12))
  (pad 1 smd roundrect (at -1.4 0) (size 1.25 1.75) (layers F.Cu F.Paste F.Mask) (roundrect_rratio 0.2) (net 10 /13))
  (pad 2 smd roundrect (at 1.4 0) (size 1.25 1.75) (layers F.Cu F.Paste F.Mask) (roundrect_rratio 0.2) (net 9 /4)))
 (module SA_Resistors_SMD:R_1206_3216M (layer F.Cu) (at 125.73 73.66)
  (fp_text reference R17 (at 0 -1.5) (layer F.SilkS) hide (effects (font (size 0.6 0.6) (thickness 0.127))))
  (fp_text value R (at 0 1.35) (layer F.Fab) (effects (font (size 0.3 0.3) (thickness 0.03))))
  (fp_line (start -0.602064 0.91) (end 0.602064 0.91) (layer F.SilkS) (width 0.12))
  (fp_line (start -0.602064 -0.91) (end 0.602064 -0.91) (layer F.SilkS) (width 0.12))
  (pad 2 smd roundrect (at 1.4 0) (size 1.25 1.75) (layers F.Cu F.Paste F.Mask) (roundrect_rratio 0.2) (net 8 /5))
  (pad 1 smd roundrect (at -1.4 0) (size 1.25 1.75) (layers F.Cu F.Paste F.Mask) (roundrect_rratio 0.2) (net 7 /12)))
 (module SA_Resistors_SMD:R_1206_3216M (layer F.Cu) (at 125.73 76.2)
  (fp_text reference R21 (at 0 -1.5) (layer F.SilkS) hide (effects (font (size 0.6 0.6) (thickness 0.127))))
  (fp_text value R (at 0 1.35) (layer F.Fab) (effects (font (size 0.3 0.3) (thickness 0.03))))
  (fp_line (start -0.602064 -0.91) (end 0.602064 -0.91) (layer F.SilkS) (width 0.12))
  (fp_line (start -0.602064 0.91) (end 0.602064 0.91) (layer F.SilkS) (width 0.12))
  (pad 1 smd roundrect (at -1.4 0) (size 1.25 1.75) (layers F.Cu F.Paste F.Mask) (roundrect_rratio 0.2) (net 6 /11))
  (pad 2 smd roundrect (at 1.4 0) (size 1.25 1.75) (layers F.Cu F.Paste F.Mask) (roundrect_rratio 0.2) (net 5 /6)))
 (gr_line (start 130.683 81.788) (end 130.683 62.992) (layer Edge.Cuts) (width 0.15))
 (gr_line (start 121.412 82.423) (end 130.048 82.423) (layer Edge.Cuts) (width 0.15))
 (gr_line (start 120.777 62.992) (end 120.777 81.788) (layer Edge.Cuts) (width 0.15))
 (gr_line (start 130.048 62.357) (end 121.412 62.357) (layer Edge.Cuts) (width 0.15))
 (gr_arc (start 130.048 62.992) (end 130.683 62.992) (angle -90) (layer Edge.Cuts) (width 0.15))
 (gr_arc (start 130.048 81.788) (end 130.048 82.423) (angle -90) (layer Edge.Cuts) (width 0.15))
 (gr_arc (start 121.412 81.788) (end 120.777 81.788) (angle -90) (layer Edge.Cuts) (width 0.15))
 (gr_arc (start 121.412 62.992) (end 121.412 62.357) (angle -90) (layer Edge.Cuts) (width 0.15))
 (segment (start 124.7925 68.58) (end 121.92 68.58) (width 0.25) (layer F.Cu) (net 11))
 (segment (start 123.73 68.58) (end 121.92 68.58) (width 0.25) (layer B.Cu) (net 11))
 (segment (start 126.6675 68.58) (end 129.54 68.58) (width 0.25) (layer F.Cu) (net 12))
 (segment (start 127.73 68.58) (end 129.54 68.58) (width 0.25) (layer B.Cu) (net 12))
 (segment (start 126.5175 71.12) (end 129.54 71.12) (width 0.25) (layer F.Cu) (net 9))
 (segment (start 127.73 71.12) (end 129.54 71.12) (width 0.25) (layer B.Cu) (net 9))
 (segment (start 124.7925 71.12) (end 121.92 71.12) (width 0.25) (layer F.Cu) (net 10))
 (segment (start 123.73 71.12) (end 121.92 71.12) (width 0.25) (layer B.Cu) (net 10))
 (segment (start 124.7925 63.5) (end 121.92 63.5) (width 0.25) (layer F.Cu) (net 16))
 (segment (start 123.73 63.5) (end 121.92 63.5) (width 0.25) (layer B.Cu) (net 16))
 (segment (start 123.73 63.5) (end 124.63 63.5) (width 0.25) (layer B.Cu) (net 16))
 (segment (start 126.6675 63.5) (end 129.54 63.5) (width 0.25) (layer F.Cu) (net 15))
 (segment (start 126.5175 63.5) (end 129.54 63.5) (width 0.25) (layer F.Cu) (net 15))
 (segment (start 127.73 63.5) (end 129.54 63.5) (width 0.25) (layer B.Cu) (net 15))
 (segment (start 126.6675 66.04) (end 129.54 66.04) (width 0.25) (layer F.Cu) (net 13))
 (segment (start 127.73 66.04) (end 129.54 66.04) (width 0.25) (layer B.Cu) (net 13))
 (segment (start 124.7925 66.04) (end 121.92 66.04) (width 0.25) (layer F.Cu) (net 14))
 (segment (start 123.73 66.04) (end 124.63 66.04) (width 0.25) (layer B.Cu) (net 14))
 (segment (start 123.73 66.04) (end 121.92 66.04) (width 0.25) (layer B.Cu) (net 14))
 (segment (start 126.6675 73.66) (end 129.54 73.66) (width 0.25) (layer F.Cu) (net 8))
 (segment (start 127.73 73.66) (end 129.54 73.66) (width 0.25) (layer B.Cu) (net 8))
 (segment (start 126.6675 76.2) (end 129.54 76.2) (width 0.25) (layer F.Cu) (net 5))
 (segment (start 127.73 76.2) (end 129.54 76.2) (width 0.25) (layer B.Cu) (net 5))
 (segment (start 127.13 78.74) (end 129.54 78.74) (width 0.25) (layer F.Cu) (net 3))
 (segment (start 127.73 78.74) (end 129.54 78.74) (width 0.25) (layer B.Cu) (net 3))
 (segment (start 126.6675 81.28) (end 129.54 81.28) (width 0.25) (layer F.Cu) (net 2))
 (segment (start 127.73 81.28) (end 129.54 81.28) (width 0.25) (layer B.Cu) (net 2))
 (segment (start 124.9425 81.28) (end 121.92 81.28) (width 0.25) (layer F.Cu) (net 1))
 (segment (start 123.73 81.28) (end 121.92 81.28) (width 0.25) (layer B.Cu) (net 1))
 (segment (start 124.7925 78.74) (end 121.92 78.74) (width 0.25) (layer F.Cu) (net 4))
 (segment (start 123.73 78.74) (end 121.92 78.74) (width 0.25) (layer B.Cu) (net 4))
 (segment (start 124.7925 76.2) (end 121.92 76.2) (width 0.25) (layer F.Cu) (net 6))
 (segment (start 123.73 76.2) (end 121.92 76.2) (width 0.25) (layer B.Cu) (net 6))
 (segment (start 124.7925 73.66) (end 121.92 73.66) (width 0.25) (layer F.Cu) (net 7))
 (segment (start 123.73 73.66) (end 121.92 73.66) (width 0.25) (layer B.Cu) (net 7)))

